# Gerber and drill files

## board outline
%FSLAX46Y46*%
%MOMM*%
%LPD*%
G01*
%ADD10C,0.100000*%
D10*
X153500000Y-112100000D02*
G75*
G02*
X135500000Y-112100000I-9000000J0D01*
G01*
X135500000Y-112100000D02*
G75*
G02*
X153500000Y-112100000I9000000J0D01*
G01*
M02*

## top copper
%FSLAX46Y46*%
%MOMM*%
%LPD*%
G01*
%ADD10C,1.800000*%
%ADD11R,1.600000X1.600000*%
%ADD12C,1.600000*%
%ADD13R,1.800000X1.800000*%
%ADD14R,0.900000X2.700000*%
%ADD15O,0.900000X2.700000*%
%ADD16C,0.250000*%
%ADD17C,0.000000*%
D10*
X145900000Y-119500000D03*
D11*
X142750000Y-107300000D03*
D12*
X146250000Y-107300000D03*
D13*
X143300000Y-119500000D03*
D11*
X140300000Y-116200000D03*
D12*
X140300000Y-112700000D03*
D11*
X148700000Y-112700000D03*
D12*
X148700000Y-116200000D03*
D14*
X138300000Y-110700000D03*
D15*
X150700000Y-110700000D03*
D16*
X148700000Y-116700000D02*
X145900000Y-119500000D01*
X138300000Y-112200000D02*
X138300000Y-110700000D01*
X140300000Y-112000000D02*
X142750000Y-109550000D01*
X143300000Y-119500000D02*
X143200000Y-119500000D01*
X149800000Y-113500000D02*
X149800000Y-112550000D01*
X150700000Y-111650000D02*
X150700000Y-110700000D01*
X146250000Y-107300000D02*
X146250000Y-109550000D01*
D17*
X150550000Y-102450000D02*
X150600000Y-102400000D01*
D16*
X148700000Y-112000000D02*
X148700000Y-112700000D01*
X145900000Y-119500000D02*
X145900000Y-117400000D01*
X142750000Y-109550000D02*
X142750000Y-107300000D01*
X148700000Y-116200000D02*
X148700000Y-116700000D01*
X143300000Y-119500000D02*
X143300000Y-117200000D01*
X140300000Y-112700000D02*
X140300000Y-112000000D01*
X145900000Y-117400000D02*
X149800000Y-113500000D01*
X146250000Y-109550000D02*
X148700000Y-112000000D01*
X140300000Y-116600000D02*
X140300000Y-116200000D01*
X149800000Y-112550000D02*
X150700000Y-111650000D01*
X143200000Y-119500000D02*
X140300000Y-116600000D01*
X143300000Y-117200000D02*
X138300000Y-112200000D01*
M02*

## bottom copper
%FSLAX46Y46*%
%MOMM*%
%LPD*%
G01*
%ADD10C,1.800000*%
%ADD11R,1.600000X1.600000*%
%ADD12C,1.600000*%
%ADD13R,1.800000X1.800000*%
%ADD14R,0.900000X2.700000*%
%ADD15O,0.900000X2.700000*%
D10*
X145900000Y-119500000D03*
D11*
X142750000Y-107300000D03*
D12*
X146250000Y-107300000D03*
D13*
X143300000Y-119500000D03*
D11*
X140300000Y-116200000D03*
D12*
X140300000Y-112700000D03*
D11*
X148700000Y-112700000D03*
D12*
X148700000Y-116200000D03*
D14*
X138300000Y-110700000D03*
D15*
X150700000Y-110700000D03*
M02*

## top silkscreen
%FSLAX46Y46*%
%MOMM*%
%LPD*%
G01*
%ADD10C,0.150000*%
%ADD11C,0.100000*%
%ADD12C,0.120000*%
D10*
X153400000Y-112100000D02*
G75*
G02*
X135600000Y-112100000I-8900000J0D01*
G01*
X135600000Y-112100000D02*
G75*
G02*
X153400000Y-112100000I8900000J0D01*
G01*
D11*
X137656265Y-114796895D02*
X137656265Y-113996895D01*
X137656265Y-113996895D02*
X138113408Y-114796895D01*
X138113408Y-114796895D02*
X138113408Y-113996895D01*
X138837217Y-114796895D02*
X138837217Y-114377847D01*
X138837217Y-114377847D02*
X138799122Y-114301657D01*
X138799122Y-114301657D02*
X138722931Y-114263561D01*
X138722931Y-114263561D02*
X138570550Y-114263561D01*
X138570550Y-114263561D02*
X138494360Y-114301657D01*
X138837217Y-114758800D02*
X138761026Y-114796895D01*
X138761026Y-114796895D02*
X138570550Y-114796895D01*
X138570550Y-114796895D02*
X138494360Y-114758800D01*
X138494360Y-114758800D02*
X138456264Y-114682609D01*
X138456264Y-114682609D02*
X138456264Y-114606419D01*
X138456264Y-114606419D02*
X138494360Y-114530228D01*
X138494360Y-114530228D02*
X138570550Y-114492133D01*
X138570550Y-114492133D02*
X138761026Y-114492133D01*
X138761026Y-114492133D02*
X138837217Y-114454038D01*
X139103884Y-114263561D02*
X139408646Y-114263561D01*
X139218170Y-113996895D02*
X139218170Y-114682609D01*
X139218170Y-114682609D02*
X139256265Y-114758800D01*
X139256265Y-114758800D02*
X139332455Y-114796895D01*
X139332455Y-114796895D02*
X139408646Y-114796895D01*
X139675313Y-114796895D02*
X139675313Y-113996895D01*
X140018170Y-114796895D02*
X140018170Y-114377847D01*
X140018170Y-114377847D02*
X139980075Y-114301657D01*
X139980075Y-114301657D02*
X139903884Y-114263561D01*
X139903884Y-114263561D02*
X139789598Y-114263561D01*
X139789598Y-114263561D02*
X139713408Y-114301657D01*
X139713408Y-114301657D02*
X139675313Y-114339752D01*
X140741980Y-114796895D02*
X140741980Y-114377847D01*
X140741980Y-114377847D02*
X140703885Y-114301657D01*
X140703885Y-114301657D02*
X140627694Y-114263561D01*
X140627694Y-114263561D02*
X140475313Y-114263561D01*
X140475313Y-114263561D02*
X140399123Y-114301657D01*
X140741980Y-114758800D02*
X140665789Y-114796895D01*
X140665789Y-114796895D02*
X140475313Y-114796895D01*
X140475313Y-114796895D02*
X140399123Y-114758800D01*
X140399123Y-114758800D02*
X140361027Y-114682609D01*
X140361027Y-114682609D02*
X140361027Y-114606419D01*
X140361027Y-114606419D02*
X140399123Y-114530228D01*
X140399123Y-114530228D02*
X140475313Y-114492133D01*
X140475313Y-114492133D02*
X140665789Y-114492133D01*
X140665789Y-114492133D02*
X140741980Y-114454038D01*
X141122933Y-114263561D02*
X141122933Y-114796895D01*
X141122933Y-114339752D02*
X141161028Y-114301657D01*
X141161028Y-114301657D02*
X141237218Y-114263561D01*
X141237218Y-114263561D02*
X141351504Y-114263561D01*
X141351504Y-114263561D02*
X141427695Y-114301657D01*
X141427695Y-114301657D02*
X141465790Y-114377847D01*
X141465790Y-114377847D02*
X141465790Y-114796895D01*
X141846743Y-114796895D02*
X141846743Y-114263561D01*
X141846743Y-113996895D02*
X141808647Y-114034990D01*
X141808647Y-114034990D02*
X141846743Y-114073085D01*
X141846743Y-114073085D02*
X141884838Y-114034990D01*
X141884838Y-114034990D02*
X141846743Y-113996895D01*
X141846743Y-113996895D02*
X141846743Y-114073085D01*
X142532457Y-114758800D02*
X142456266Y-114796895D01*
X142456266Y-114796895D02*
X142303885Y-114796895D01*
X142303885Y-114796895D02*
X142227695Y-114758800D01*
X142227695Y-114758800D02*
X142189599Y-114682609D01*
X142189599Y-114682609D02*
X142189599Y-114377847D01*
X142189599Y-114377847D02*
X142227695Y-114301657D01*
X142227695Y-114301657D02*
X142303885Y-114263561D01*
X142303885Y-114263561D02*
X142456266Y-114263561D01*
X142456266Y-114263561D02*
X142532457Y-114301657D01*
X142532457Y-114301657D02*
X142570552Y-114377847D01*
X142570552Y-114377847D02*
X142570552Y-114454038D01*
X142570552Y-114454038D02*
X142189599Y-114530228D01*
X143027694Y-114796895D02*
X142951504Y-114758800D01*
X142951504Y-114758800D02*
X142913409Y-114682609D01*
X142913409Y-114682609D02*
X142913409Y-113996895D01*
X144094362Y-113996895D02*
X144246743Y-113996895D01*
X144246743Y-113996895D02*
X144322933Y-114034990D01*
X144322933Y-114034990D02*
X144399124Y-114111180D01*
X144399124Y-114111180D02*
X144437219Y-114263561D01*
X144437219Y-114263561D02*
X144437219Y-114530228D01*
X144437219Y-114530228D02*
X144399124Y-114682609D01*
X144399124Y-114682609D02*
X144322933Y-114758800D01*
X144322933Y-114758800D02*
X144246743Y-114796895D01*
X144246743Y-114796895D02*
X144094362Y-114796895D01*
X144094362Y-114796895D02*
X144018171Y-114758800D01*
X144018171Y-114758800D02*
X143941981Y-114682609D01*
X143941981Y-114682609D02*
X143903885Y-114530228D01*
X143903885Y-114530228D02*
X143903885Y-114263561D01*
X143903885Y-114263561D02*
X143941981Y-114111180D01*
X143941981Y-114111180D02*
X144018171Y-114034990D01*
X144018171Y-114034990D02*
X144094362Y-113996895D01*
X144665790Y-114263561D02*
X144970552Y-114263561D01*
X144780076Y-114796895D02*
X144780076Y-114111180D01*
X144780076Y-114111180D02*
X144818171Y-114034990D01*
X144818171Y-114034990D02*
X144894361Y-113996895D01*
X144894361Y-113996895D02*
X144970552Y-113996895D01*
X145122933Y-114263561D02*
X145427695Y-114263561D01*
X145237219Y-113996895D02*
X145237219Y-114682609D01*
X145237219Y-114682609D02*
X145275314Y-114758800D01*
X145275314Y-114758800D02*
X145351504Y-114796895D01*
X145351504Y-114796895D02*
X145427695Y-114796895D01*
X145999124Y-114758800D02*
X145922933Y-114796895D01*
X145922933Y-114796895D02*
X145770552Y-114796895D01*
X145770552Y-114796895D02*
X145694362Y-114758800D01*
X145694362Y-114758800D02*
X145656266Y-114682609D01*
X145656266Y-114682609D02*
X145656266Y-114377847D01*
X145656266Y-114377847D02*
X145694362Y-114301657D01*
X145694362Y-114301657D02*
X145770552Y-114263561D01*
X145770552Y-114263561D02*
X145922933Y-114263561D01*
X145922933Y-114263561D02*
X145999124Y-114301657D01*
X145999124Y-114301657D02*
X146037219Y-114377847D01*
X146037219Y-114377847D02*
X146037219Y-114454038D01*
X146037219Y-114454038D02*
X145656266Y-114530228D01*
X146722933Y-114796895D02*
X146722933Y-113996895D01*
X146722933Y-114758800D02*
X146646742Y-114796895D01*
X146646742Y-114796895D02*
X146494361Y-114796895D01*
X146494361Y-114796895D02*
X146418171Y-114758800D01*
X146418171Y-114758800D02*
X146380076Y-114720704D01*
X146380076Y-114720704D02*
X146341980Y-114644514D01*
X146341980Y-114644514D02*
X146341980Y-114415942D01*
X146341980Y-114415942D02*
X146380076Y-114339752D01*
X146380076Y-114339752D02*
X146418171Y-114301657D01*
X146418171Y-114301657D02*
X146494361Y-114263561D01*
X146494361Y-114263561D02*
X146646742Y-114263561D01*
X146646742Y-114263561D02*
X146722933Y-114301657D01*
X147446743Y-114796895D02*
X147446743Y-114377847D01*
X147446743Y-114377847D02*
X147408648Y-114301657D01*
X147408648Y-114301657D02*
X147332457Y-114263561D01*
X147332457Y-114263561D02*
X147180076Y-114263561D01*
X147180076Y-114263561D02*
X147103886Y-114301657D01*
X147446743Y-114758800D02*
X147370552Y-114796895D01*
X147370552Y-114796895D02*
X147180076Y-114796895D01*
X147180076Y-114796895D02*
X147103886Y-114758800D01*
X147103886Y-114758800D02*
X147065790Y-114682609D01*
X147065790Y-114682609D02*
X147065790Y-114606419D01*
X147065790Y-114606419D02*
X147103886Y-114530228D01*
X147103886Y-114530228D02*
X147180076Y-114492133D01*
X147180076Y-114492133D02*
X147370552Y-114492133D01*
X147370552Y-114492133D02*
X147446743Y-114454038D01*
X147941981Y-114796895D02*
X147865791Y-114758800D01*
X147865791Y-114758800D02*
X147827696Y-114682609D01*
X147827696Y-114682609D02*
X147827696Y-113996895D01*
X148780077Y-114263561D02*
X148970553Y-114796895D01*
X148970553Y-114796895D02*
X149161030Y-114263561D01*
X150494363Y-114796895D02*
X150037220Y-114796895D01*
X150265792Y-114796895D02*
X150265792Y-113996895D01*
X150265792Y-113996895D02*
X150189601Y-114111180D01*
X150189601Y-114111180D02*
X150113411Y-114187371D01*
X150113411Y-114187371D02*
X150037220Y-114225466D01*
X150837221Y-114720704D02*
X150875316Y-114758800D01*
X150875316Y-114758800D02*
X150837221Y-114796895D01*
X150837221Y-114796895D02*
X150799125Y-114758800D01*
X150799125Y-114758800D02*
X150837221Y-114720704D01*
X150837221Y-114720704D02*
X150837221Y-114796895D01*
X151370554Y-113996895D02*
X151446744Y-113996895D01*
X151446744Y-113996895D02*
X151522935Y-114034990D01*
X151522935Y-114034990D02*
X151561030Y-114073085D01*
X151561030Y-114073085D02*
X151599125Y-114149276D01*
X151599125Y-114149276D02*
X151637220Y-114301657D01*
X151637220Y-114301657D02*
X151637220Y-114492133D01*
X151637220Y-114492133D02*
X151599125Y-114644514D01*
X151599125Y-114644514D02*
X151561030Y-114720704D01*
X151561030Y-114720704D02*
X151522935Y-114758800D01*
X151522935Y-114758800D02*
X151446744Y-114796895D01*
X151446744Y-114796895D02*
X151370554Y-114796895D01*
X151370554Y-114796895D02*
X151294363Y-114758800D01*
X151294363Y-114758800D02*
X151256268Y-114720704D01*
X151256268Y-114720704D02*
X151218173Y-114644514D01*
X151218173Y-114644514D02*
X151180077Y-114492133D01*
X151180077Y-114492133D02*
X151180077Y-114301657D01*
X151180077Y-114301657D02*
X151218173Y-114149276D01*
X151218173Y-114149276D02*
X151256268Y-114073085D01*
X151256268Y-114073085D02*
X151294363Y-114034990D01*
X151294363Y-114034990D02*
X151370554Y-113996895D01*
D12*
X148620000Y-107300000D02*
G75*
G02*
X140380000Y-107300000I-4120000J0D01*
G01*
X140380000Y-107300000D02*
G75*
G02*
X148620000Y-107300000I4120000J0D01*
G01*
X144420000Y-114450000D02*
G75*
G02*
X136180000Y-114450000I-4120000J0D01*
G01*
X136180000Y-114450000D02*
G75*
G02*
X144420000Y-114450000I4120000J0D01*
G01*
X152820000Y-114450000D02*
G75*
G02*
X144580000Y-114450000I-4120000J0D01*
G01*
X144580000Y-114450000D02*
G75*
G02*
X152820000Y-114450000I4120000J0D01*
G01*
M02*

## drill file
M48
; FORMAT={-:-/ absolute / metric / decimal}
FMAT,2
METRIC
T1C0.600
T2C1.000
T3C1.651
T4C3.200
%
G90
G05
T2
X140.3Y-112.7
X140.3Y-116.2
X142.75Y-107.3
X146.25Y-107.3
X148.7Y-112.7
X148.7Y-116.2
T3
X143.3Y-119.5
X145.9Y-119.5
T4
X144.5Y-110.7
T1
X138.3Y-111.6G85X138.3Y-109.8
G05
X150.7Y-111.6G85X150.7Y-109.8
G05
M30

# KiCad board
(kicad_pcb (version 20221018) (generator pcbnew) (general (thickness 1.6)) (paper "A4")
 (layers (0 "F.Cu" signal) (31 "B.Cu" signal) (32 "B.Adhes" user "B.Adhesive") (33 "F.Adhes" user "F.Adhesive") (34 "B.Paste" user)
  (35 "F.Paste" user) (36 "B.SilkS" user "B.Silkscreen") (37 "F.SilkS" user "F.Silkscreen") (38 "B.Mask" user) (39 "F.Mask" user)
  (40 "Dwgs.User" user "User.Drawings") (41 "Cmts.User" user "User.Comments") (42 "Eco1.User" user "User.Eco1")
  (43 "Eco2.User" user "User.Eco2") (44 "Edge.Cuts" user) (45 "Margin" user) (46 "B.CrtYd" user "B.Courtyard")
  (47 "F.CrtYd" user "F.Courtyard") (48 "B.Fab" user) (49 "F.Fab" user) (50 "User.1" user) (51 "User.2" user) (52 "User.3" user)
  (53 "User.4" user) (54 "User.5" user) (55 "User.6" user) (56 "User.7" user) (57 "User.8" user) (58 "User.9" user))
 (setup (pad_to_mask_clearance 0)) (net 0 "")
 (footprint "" (layer "F.Cu") (at 145.9 119.5)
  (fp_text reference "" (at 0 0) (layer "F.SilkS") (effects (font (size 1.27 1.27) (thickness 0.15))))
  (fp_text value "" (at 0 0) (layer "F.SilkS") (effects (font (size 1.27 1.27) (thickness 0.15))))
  (pad "2" thru_hole circle (at 0 0) (size 1.8 1.8) (drill 1.651) (layers "*.Cu" "*.Mask")))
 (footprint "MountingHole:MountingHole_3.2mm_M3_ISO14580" (layer "F.Cu") (at 144.5 110.7)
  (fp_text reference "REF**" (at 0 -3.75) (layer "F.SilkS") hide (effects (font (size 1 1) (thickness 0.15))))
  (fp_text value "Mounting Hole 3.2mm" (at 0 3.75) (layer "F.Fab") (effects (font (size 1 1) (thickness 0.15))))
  (pad "" np_thru_hole circle (at 0 0) (size 3.2 3.2) (drill 3.2) (layers "F&B.Cu" "*.Mask" "B.Paste")))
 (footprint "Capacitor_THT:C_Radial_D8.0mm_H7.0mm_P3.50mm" (layer "F.Cu") (at 142.75 107.3)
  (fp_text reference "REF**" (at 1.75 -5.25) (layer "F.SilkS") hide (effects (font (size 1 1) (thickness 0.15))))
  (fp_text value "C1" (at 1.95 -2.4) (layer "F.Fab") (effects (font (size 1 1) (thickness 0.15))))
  (fp_circle (center 1.75 0) (end 5.87 0) (stroke (width 0.12) (type solid)) (fill none) (layer "F.SilkS"))
  (pad "1" thru_hole rect (at 0 0) (size 1.6 1.6) (drill 1) (layers "*.Cu" "*.Mask"))
  (pad "2" thru_hole circle (at 3.5 0) (size 1.6 1.6) (drill 1) (layers "*.Cu" "*.Mask")))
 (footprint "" (layer "F.Cu") (at 143.3 119.5)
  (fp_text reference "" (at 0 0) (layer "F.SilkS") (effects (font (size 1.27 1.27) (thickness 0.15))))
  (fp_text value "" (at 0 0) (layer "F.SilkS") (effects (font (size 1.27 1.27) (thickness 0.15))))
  (pad "1" thru_hole rect (at 0 0) (size 1.8 1.8) (drill 1.651) (layers "*.Cu" "*.Mask")))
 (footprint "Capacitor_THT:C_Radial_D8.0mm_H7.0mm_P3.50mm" (layer "F.Cu") (at 140.3 116.2 90)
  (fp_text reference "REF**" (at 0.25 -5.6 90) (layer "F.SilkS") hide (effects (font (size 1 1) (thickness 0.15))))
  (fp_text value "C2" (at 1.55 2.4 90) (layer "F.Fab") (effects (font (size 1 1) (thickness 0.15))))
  (fp_circle (center 1.75 0) (end 5.87 0) (stroke (width 0.12) (type solid)) (fill none) (layer "F.SilkS"))
  (pad "1" thru_hole rect (at 0 0 90) (size 1.6 1.6) (drill 1) (layers "*.Cu" "*.Mask"))
  (pad "2" thru_hole circle (at 3.5 0 90) (size 1.6 1.6) (drill 1) (layers "*.Cu" "*.Mask")))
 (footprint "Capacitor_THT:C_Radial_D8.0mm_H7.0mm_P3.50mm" (layer "F.Cu") (at 148.7 112.7 -90)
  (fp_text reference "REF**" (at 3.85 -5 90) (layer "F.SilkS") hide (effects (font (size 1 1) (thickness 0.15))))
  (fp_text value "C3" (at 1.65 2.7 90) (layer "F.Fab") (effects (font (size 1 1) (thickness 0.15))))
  (fp_circle (center 1.75 0) (end 5.87 0) (stroke (width 0.12) (type solid)) (fill none) (layer "F.SilkS"))
  (pad "1" thru_hole rect (at 0 0 270) (size 1.6 1.6) (drill 1) (layers "*.Cu" "*.Mask"))
  (pad "2" thru_hole circle (at 3.5 0 270) (size 1.6 1.6) (drill 1) (layers "*.Cu" "*.Mask")))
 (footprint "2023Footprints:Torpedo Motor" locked (layer "B.Cu") (at 144.5 110.7 90)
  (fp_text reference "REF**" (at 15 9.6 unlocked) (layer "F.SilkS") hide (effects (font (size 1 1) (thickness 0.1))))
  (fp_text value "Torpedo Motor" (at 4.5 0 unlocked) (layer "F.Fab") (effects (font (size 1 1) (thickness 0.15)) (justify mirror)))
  (pad "1" thru_hole rect locked (at 0 -6.2 90) (size 2.7 0.9) (drill oval 2.4 0.6) (layers "*.Cu" "*.Mask"))
  (pad "2" thru_hole oval locked (at 0 6.2 90) (size 2.7 0.9) (drill oval 2.4 0.6) (layers "*.Cu" "*.Mask")))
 (gr_circle (center 144.5 112.1) (end 153.4 112.1) (stroke (width 0.15) (type default)) (fill none) (layer "F.SilkS"))
 (gr_circle (center 144.5 112.1) (end 153.5 112.1) (stroke (width 0.1) (type default)) (fill none) (layer "Edge.Cuts"))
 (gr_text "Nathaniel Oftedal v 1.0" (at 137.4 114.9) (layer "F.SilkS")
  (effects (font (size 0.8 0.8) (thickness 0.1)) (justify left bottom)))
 (segment (start 148.7 116.7) (end 145.9 119.5) (width 0.25) (layer "F.Cu") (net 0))
 (segment (start 138.3 112.2) (end 138.3 110.7) (width 0.25) (layer "F.Cu") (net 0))
 (segment (start 140.3 112) (end 142.75 109.55) (width 0.25) (layer "F.Cu") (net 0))
 (segment (start 143.3 119.5) (end 143.2 119.5) (width 0.25) (layer "F.Cu") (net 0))
 (segment (start 149.8 113.5) (end 149.8 112.55) (width 0.25) (layer "F.Cu") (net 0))
 (segment (start 150.7 111.65) (end 150.7 110.7) (width 0.25) (layer "F.Cu") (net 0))
 (segment (start 146.25 107.3) (end 146.25 109.55) (width 0.25) (layer "F.Cu") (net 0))
 (segment (start 150.55 102.45) (end 150.6 102.4) (width 0) (layer "F.Cu") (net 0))
 (segment (start 148.7 112) (end 148.7 112.7) (width 0.25) (layer "F.Cu") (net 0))
 (segment (start 145.9 119.5) (end 145.9 117.4) (width 0.25) (layer "F.Cu") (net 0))
 (segment (start 142.75 109.55) (end 142.75 107.3) (width 0.25) (layer "F.Cu") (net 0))
 (segment (start 148.7 116.2) (end 148.7 116.7) (width 0.25) (layer "F.Cu") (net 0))
 (segment (start 143.3 119.5) (end 143.3 117.2) (width 0.25) (layer "F.Cu") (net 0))
 (segment (start 140.3 112.7) (end 140.3 112) (width 0.25) (layer "F.Cu") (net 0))
 (segment (start 145.9 117.4) (end 149.8 113.5) (width 0.25) (layer "F.Cu") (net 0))
 (segment (start 146.25 109.55) (end 148.7 112) (width 0.25) (layer "F.Cu") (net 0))
 (segment (start 140.3 116.6) (end 140.3 116.2) (width 0.25) (layer "F.Cu") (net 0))
 (segment (start 149.8 112.55) (end 150.7 111.65) (width 0.25) (layer "F.Cu") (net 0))
 (segment (start 143.2 119.5) (end 140.3 116.6) (width 0.25) (layer "F.Cu") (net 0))
 (segment (start 143.3 117.2) (end 138.3 112.2) (width 0.25) (layer "F.Cu") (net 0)))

